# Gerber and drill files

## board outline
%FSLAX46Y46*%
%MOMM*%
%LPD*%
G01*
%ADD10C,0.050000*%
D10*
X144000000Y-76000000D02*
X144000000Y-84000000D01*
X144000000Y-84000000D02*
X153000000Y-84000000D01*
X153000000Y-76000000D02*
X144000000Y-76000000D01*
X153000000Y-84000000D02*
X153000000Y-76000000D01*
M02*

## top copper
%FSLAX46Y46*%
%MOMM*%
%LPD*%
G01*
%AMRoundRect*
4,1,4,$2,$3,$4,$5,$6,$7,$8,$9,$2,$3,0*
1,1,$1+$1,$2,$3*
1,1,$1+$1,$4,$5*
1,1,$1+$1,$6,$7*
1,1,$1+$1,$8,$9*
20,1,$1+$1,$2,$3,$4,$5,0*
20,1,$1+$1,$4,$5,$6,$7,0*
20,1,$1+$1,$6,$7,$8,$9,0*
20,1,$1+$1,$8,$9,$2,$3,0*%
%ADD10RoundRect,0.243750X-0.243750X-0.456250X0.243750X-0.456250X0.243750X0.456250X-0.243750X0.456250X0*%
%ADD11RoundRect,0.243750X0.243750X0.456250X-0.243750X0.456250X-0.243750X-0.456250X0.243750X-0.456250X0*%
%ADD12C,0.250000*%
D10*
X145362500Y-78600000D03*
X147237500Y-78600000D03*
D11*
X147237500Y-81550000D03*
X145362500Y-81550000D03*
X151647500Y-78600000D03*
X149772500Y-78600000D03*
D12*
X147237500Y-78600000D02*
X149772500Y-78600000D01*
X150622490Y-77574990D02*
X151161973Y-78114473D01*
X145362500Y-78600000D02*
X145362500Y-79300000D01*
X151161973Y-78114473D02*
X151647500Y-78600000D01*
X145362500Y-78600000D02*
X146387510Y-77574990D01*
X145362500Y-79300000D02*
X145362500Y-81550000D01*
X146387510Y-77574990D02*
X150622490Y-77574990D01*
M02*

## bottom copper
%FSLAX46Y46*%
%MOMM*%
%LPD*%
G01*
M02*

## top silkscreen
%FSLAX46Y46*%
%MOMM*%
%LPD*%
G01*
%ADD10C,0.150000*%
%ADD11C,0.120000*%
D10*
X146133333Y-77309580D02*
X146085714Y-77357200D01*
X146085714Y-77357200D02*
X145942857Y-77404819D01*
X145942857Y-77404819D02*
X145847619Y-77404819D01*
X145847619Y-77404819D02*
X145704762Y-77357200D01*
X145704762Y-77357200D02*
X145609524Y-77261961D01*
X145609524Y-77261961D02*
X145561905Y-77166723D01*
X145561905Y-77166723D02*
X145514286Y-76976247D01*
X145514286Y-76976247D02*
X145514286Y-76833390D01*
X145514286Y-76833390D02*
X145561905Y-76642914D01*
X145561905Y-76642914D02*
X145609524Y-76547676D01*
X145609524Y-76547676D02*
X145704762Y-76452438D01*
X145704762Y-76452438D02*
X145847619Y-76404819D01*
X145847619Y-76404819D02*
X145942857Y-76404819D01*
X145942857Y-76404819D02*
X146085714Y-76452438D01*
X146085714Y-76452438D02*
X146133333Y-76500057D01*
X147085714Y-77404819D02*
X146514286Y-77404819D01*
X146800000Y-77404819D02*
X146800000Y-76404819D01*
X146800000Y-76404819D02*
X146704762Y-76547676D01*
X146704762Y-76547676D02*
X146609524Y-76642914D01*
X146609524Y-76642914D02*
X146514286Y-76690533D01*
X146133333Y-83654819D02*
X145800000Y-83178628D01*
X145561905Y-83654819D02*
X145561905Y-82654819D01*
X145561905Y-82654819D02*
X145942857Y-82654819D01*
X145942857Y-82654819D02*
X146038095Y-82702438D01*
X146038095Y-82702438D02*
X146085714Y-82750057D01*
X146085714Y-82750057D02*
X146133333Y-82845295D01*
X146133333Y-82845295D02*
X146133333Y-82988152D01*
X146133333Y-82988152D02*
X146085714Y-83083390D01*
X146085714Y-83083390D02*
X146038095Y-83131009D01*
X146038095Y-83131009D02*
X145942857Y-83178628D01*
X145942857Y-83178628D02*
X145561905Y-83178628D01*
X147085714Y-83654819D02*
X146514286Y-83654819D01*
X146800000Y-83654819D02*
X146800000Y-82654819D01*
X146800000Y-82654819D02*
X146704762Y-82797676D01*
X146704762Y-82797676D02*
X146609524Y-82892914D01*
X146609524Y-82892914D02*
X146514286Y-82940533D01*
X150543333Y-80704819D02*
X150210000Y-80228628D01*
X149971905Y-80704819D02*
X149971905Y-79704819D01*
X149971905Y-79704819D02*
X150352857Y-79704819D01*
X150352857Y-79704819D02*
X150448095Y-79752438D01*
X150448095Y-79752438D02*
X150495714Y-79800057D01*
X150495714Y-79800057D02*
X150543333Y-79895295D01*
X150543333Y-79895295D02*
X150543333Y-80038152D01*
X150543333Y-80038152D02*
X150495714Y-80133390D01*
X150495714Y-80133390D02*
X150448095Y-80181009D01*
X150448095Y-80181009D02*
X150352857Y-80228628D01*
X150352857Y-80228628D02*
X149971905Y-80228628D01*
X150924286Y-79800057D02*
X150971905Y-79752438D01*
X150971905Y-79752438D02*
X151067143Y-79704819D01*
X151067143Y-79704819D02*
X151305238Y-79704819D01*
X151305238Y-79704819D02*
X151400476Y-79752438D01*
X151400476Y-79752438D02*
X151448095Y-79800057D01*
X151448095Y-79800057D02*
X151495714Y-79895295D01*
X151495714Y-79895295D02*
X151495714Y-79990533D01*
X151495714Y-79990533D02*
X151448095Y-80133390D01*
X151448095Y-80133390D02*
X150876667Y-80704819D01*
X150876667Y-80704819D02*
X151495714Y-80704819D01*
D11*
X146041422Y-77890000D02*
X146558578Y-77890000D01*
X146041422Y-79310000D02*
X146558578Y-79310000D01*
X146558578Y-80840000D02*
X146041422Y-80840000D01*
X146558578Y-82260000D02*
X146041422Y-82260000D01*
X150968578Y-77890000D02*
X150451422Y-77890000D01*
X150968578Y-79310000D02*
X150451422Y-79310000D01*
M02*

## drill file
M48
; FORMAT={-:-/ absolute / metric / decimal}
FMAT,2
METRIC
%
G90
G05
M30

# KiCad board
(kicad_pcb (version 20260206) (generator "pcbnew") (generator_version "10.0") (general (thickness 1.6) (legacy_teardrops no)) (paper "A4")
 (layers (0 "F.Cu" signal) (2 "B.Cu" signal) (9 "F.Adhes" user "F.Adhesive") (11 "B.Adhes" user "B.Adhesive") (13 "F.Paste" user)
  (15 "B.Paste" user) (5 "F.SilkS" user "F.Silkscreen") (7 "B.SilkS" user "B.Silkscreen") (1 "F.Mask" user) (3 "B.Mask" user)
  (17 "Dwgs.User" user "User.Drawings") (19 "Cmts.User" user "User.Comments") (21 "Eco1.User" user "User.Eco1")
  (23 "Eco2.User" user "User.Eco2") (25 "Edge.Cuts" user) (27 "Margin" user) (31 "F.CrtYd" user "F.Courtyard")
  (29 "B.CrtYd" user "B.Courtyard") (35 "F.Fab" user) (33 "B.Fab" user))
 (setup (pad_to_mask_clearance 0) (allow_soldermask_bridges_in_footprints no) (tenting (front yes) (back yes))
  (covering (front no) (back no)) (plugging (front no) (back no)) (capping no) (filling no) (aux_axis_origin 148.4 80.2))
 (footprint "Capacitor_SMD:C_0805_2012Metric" (layer "F.Cu") (at 146.3 78.6)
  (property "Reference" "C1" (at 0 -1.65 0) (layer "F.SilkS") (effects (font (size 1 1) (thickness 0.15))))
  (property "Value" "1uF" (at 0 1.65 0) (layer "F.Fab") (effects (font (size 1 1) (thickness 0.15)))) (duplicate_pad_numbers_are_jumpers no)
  (fp_line (start -0.258578 -0.71) (end 0.258578 -0.71) (stroke (width 0.12) (type solid)) (layer "F.SilkS"))
  (fp_line (start -0.258578 0.71) (end 0.258578 0.71) (stroke (width 0.12) (type solid)) (layer "F.SilkS"))
  (pad "1" smd roundrect (at -0.9375 0) (size 0.975 1.4) (layers "F.Cu" "F.Mask" "F.Paste") (roundrect_rratio 0.25) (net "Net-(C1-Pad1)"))
  (pad "2" smd roundrect (at 0.9375 0) (size 0.975 1.4) (layers "F.Cu" "F.Mask" "F.Paste") (roundrect_rratio 0.25) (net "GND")))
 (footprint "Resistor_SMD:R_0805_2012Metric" (layer "F.Cu") (at 146.3 81.55 180)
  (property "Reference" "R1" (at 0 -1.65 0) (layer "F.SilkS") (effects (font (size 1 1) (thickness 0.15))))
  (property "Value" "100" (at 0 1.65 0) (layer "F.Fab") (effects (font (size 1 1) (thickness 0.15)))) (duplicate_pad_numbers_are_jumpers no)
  (fp_line (start -0.258578 0.71) (end 0.258578 0.71) (stroke (width 0.12) (type solid)) (layer "F.SilkS"))
  (fp_line (start -0.258578 -0.71) (end 0.258578 -0.71) (stroke (width 0.12) (type solid)) (layer "F.SilkS"))
  (pad "1" smd roundrect (at -0.9375 0 180) (size 0.975 1.4) (layers "F.Cu" "F.Mask" "F.Paste") (roundrect_rratio 0.25) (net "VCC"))
  (pad "2" smd roundrect (at 0.9375 0 180) (size 0.975 1.4) (layers "F.Cu" "F.Mask" "F.Paste") (roundrect_rratio 0.25) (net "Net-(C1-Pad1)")))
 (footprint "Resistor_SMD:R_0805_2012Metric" (layer "F.Cu") (at 150.71 78.6 180)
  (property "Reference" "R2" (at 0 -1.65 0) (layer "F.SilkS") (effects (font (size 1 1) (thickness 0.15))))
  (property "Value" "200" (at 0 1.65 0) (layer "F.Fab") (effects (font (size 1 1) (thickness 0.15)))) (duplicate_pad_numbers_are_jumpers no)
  (fp_line (start -0.258578 0.71) (end 0.258578 0.71) (stroke (width 0.12) (type solid)) (layer "F.SilkS"))
  (fp_line (start -0.258578 -0.71) (end 0.258578 -0.71) (stroke (width 0.12) (type solid)) (layer "F.SilkS"))
  (pad "1" smd roundrect (at -0.9375 0 180) (size 0.975 1.4) (layers "F.Cu" "F.Mask" "F.Paste") (roundrect_rratio 0.25)
   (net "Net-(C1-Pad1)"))
  (pad "2" smd roundrect (at 0.9375 0 180) (size 0.975 1.4) (layers "F.Cu" "F.Mask" "F.Paste") (roundrect_rratio 0.25) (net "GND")))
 (gr_line (start 144 76) (end 144 84) (stroke (width 0.05) (type solid)) (layer "Edge.Cuts"))
 (gr_line (start 144 84) (end 153 84) (stroke (width 0.05) (type solid)) (layer "Edge.Cuts"))
 (gr_line (start 153 76) (end 144 76) (stroke (width 0.05) (type solid)) (layer "Edge.Cuts"))
 (gr_line (start 153 84) (end 153 76) (stroke (width 0.05) (type solid)) (layer "Edge.Cuts"))
 (segment (start 147.2375 78.6) (end 149.7725 78.6) (width 0.25) (layer "F.Cu") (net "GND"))
 (segment (start 150.62249 77.57499) (end 151.161973 78.114473) (width 0.25) (layer "F.Cu") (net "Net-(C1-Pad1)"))
 (segment (start 145.3625 78.6) (end 145.3625 79.3) (width 0.25) (layer "F.Cu") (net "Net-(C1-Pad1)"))
 (segment (start 151.161973 78.114473) (end 151.6475 78.6) (width 0.25) (layer "F.Cu") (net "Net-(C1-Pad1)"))
 (segment (start 145.3625 78.6) (end 146.38751 77.57499) (width 0.25) (layer "F.Cu") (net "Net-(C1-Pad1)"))
 (segment (start 145.3625 79.3) (end 145.3625 81.55) (width 0.25) (layer "F.Cu") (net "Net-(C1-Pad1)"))
 (segment (start 146.38751 77.57499) (end 150.62249 77.57499) (width 0.25) (layer "F.Cu") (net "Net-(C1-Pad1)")))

